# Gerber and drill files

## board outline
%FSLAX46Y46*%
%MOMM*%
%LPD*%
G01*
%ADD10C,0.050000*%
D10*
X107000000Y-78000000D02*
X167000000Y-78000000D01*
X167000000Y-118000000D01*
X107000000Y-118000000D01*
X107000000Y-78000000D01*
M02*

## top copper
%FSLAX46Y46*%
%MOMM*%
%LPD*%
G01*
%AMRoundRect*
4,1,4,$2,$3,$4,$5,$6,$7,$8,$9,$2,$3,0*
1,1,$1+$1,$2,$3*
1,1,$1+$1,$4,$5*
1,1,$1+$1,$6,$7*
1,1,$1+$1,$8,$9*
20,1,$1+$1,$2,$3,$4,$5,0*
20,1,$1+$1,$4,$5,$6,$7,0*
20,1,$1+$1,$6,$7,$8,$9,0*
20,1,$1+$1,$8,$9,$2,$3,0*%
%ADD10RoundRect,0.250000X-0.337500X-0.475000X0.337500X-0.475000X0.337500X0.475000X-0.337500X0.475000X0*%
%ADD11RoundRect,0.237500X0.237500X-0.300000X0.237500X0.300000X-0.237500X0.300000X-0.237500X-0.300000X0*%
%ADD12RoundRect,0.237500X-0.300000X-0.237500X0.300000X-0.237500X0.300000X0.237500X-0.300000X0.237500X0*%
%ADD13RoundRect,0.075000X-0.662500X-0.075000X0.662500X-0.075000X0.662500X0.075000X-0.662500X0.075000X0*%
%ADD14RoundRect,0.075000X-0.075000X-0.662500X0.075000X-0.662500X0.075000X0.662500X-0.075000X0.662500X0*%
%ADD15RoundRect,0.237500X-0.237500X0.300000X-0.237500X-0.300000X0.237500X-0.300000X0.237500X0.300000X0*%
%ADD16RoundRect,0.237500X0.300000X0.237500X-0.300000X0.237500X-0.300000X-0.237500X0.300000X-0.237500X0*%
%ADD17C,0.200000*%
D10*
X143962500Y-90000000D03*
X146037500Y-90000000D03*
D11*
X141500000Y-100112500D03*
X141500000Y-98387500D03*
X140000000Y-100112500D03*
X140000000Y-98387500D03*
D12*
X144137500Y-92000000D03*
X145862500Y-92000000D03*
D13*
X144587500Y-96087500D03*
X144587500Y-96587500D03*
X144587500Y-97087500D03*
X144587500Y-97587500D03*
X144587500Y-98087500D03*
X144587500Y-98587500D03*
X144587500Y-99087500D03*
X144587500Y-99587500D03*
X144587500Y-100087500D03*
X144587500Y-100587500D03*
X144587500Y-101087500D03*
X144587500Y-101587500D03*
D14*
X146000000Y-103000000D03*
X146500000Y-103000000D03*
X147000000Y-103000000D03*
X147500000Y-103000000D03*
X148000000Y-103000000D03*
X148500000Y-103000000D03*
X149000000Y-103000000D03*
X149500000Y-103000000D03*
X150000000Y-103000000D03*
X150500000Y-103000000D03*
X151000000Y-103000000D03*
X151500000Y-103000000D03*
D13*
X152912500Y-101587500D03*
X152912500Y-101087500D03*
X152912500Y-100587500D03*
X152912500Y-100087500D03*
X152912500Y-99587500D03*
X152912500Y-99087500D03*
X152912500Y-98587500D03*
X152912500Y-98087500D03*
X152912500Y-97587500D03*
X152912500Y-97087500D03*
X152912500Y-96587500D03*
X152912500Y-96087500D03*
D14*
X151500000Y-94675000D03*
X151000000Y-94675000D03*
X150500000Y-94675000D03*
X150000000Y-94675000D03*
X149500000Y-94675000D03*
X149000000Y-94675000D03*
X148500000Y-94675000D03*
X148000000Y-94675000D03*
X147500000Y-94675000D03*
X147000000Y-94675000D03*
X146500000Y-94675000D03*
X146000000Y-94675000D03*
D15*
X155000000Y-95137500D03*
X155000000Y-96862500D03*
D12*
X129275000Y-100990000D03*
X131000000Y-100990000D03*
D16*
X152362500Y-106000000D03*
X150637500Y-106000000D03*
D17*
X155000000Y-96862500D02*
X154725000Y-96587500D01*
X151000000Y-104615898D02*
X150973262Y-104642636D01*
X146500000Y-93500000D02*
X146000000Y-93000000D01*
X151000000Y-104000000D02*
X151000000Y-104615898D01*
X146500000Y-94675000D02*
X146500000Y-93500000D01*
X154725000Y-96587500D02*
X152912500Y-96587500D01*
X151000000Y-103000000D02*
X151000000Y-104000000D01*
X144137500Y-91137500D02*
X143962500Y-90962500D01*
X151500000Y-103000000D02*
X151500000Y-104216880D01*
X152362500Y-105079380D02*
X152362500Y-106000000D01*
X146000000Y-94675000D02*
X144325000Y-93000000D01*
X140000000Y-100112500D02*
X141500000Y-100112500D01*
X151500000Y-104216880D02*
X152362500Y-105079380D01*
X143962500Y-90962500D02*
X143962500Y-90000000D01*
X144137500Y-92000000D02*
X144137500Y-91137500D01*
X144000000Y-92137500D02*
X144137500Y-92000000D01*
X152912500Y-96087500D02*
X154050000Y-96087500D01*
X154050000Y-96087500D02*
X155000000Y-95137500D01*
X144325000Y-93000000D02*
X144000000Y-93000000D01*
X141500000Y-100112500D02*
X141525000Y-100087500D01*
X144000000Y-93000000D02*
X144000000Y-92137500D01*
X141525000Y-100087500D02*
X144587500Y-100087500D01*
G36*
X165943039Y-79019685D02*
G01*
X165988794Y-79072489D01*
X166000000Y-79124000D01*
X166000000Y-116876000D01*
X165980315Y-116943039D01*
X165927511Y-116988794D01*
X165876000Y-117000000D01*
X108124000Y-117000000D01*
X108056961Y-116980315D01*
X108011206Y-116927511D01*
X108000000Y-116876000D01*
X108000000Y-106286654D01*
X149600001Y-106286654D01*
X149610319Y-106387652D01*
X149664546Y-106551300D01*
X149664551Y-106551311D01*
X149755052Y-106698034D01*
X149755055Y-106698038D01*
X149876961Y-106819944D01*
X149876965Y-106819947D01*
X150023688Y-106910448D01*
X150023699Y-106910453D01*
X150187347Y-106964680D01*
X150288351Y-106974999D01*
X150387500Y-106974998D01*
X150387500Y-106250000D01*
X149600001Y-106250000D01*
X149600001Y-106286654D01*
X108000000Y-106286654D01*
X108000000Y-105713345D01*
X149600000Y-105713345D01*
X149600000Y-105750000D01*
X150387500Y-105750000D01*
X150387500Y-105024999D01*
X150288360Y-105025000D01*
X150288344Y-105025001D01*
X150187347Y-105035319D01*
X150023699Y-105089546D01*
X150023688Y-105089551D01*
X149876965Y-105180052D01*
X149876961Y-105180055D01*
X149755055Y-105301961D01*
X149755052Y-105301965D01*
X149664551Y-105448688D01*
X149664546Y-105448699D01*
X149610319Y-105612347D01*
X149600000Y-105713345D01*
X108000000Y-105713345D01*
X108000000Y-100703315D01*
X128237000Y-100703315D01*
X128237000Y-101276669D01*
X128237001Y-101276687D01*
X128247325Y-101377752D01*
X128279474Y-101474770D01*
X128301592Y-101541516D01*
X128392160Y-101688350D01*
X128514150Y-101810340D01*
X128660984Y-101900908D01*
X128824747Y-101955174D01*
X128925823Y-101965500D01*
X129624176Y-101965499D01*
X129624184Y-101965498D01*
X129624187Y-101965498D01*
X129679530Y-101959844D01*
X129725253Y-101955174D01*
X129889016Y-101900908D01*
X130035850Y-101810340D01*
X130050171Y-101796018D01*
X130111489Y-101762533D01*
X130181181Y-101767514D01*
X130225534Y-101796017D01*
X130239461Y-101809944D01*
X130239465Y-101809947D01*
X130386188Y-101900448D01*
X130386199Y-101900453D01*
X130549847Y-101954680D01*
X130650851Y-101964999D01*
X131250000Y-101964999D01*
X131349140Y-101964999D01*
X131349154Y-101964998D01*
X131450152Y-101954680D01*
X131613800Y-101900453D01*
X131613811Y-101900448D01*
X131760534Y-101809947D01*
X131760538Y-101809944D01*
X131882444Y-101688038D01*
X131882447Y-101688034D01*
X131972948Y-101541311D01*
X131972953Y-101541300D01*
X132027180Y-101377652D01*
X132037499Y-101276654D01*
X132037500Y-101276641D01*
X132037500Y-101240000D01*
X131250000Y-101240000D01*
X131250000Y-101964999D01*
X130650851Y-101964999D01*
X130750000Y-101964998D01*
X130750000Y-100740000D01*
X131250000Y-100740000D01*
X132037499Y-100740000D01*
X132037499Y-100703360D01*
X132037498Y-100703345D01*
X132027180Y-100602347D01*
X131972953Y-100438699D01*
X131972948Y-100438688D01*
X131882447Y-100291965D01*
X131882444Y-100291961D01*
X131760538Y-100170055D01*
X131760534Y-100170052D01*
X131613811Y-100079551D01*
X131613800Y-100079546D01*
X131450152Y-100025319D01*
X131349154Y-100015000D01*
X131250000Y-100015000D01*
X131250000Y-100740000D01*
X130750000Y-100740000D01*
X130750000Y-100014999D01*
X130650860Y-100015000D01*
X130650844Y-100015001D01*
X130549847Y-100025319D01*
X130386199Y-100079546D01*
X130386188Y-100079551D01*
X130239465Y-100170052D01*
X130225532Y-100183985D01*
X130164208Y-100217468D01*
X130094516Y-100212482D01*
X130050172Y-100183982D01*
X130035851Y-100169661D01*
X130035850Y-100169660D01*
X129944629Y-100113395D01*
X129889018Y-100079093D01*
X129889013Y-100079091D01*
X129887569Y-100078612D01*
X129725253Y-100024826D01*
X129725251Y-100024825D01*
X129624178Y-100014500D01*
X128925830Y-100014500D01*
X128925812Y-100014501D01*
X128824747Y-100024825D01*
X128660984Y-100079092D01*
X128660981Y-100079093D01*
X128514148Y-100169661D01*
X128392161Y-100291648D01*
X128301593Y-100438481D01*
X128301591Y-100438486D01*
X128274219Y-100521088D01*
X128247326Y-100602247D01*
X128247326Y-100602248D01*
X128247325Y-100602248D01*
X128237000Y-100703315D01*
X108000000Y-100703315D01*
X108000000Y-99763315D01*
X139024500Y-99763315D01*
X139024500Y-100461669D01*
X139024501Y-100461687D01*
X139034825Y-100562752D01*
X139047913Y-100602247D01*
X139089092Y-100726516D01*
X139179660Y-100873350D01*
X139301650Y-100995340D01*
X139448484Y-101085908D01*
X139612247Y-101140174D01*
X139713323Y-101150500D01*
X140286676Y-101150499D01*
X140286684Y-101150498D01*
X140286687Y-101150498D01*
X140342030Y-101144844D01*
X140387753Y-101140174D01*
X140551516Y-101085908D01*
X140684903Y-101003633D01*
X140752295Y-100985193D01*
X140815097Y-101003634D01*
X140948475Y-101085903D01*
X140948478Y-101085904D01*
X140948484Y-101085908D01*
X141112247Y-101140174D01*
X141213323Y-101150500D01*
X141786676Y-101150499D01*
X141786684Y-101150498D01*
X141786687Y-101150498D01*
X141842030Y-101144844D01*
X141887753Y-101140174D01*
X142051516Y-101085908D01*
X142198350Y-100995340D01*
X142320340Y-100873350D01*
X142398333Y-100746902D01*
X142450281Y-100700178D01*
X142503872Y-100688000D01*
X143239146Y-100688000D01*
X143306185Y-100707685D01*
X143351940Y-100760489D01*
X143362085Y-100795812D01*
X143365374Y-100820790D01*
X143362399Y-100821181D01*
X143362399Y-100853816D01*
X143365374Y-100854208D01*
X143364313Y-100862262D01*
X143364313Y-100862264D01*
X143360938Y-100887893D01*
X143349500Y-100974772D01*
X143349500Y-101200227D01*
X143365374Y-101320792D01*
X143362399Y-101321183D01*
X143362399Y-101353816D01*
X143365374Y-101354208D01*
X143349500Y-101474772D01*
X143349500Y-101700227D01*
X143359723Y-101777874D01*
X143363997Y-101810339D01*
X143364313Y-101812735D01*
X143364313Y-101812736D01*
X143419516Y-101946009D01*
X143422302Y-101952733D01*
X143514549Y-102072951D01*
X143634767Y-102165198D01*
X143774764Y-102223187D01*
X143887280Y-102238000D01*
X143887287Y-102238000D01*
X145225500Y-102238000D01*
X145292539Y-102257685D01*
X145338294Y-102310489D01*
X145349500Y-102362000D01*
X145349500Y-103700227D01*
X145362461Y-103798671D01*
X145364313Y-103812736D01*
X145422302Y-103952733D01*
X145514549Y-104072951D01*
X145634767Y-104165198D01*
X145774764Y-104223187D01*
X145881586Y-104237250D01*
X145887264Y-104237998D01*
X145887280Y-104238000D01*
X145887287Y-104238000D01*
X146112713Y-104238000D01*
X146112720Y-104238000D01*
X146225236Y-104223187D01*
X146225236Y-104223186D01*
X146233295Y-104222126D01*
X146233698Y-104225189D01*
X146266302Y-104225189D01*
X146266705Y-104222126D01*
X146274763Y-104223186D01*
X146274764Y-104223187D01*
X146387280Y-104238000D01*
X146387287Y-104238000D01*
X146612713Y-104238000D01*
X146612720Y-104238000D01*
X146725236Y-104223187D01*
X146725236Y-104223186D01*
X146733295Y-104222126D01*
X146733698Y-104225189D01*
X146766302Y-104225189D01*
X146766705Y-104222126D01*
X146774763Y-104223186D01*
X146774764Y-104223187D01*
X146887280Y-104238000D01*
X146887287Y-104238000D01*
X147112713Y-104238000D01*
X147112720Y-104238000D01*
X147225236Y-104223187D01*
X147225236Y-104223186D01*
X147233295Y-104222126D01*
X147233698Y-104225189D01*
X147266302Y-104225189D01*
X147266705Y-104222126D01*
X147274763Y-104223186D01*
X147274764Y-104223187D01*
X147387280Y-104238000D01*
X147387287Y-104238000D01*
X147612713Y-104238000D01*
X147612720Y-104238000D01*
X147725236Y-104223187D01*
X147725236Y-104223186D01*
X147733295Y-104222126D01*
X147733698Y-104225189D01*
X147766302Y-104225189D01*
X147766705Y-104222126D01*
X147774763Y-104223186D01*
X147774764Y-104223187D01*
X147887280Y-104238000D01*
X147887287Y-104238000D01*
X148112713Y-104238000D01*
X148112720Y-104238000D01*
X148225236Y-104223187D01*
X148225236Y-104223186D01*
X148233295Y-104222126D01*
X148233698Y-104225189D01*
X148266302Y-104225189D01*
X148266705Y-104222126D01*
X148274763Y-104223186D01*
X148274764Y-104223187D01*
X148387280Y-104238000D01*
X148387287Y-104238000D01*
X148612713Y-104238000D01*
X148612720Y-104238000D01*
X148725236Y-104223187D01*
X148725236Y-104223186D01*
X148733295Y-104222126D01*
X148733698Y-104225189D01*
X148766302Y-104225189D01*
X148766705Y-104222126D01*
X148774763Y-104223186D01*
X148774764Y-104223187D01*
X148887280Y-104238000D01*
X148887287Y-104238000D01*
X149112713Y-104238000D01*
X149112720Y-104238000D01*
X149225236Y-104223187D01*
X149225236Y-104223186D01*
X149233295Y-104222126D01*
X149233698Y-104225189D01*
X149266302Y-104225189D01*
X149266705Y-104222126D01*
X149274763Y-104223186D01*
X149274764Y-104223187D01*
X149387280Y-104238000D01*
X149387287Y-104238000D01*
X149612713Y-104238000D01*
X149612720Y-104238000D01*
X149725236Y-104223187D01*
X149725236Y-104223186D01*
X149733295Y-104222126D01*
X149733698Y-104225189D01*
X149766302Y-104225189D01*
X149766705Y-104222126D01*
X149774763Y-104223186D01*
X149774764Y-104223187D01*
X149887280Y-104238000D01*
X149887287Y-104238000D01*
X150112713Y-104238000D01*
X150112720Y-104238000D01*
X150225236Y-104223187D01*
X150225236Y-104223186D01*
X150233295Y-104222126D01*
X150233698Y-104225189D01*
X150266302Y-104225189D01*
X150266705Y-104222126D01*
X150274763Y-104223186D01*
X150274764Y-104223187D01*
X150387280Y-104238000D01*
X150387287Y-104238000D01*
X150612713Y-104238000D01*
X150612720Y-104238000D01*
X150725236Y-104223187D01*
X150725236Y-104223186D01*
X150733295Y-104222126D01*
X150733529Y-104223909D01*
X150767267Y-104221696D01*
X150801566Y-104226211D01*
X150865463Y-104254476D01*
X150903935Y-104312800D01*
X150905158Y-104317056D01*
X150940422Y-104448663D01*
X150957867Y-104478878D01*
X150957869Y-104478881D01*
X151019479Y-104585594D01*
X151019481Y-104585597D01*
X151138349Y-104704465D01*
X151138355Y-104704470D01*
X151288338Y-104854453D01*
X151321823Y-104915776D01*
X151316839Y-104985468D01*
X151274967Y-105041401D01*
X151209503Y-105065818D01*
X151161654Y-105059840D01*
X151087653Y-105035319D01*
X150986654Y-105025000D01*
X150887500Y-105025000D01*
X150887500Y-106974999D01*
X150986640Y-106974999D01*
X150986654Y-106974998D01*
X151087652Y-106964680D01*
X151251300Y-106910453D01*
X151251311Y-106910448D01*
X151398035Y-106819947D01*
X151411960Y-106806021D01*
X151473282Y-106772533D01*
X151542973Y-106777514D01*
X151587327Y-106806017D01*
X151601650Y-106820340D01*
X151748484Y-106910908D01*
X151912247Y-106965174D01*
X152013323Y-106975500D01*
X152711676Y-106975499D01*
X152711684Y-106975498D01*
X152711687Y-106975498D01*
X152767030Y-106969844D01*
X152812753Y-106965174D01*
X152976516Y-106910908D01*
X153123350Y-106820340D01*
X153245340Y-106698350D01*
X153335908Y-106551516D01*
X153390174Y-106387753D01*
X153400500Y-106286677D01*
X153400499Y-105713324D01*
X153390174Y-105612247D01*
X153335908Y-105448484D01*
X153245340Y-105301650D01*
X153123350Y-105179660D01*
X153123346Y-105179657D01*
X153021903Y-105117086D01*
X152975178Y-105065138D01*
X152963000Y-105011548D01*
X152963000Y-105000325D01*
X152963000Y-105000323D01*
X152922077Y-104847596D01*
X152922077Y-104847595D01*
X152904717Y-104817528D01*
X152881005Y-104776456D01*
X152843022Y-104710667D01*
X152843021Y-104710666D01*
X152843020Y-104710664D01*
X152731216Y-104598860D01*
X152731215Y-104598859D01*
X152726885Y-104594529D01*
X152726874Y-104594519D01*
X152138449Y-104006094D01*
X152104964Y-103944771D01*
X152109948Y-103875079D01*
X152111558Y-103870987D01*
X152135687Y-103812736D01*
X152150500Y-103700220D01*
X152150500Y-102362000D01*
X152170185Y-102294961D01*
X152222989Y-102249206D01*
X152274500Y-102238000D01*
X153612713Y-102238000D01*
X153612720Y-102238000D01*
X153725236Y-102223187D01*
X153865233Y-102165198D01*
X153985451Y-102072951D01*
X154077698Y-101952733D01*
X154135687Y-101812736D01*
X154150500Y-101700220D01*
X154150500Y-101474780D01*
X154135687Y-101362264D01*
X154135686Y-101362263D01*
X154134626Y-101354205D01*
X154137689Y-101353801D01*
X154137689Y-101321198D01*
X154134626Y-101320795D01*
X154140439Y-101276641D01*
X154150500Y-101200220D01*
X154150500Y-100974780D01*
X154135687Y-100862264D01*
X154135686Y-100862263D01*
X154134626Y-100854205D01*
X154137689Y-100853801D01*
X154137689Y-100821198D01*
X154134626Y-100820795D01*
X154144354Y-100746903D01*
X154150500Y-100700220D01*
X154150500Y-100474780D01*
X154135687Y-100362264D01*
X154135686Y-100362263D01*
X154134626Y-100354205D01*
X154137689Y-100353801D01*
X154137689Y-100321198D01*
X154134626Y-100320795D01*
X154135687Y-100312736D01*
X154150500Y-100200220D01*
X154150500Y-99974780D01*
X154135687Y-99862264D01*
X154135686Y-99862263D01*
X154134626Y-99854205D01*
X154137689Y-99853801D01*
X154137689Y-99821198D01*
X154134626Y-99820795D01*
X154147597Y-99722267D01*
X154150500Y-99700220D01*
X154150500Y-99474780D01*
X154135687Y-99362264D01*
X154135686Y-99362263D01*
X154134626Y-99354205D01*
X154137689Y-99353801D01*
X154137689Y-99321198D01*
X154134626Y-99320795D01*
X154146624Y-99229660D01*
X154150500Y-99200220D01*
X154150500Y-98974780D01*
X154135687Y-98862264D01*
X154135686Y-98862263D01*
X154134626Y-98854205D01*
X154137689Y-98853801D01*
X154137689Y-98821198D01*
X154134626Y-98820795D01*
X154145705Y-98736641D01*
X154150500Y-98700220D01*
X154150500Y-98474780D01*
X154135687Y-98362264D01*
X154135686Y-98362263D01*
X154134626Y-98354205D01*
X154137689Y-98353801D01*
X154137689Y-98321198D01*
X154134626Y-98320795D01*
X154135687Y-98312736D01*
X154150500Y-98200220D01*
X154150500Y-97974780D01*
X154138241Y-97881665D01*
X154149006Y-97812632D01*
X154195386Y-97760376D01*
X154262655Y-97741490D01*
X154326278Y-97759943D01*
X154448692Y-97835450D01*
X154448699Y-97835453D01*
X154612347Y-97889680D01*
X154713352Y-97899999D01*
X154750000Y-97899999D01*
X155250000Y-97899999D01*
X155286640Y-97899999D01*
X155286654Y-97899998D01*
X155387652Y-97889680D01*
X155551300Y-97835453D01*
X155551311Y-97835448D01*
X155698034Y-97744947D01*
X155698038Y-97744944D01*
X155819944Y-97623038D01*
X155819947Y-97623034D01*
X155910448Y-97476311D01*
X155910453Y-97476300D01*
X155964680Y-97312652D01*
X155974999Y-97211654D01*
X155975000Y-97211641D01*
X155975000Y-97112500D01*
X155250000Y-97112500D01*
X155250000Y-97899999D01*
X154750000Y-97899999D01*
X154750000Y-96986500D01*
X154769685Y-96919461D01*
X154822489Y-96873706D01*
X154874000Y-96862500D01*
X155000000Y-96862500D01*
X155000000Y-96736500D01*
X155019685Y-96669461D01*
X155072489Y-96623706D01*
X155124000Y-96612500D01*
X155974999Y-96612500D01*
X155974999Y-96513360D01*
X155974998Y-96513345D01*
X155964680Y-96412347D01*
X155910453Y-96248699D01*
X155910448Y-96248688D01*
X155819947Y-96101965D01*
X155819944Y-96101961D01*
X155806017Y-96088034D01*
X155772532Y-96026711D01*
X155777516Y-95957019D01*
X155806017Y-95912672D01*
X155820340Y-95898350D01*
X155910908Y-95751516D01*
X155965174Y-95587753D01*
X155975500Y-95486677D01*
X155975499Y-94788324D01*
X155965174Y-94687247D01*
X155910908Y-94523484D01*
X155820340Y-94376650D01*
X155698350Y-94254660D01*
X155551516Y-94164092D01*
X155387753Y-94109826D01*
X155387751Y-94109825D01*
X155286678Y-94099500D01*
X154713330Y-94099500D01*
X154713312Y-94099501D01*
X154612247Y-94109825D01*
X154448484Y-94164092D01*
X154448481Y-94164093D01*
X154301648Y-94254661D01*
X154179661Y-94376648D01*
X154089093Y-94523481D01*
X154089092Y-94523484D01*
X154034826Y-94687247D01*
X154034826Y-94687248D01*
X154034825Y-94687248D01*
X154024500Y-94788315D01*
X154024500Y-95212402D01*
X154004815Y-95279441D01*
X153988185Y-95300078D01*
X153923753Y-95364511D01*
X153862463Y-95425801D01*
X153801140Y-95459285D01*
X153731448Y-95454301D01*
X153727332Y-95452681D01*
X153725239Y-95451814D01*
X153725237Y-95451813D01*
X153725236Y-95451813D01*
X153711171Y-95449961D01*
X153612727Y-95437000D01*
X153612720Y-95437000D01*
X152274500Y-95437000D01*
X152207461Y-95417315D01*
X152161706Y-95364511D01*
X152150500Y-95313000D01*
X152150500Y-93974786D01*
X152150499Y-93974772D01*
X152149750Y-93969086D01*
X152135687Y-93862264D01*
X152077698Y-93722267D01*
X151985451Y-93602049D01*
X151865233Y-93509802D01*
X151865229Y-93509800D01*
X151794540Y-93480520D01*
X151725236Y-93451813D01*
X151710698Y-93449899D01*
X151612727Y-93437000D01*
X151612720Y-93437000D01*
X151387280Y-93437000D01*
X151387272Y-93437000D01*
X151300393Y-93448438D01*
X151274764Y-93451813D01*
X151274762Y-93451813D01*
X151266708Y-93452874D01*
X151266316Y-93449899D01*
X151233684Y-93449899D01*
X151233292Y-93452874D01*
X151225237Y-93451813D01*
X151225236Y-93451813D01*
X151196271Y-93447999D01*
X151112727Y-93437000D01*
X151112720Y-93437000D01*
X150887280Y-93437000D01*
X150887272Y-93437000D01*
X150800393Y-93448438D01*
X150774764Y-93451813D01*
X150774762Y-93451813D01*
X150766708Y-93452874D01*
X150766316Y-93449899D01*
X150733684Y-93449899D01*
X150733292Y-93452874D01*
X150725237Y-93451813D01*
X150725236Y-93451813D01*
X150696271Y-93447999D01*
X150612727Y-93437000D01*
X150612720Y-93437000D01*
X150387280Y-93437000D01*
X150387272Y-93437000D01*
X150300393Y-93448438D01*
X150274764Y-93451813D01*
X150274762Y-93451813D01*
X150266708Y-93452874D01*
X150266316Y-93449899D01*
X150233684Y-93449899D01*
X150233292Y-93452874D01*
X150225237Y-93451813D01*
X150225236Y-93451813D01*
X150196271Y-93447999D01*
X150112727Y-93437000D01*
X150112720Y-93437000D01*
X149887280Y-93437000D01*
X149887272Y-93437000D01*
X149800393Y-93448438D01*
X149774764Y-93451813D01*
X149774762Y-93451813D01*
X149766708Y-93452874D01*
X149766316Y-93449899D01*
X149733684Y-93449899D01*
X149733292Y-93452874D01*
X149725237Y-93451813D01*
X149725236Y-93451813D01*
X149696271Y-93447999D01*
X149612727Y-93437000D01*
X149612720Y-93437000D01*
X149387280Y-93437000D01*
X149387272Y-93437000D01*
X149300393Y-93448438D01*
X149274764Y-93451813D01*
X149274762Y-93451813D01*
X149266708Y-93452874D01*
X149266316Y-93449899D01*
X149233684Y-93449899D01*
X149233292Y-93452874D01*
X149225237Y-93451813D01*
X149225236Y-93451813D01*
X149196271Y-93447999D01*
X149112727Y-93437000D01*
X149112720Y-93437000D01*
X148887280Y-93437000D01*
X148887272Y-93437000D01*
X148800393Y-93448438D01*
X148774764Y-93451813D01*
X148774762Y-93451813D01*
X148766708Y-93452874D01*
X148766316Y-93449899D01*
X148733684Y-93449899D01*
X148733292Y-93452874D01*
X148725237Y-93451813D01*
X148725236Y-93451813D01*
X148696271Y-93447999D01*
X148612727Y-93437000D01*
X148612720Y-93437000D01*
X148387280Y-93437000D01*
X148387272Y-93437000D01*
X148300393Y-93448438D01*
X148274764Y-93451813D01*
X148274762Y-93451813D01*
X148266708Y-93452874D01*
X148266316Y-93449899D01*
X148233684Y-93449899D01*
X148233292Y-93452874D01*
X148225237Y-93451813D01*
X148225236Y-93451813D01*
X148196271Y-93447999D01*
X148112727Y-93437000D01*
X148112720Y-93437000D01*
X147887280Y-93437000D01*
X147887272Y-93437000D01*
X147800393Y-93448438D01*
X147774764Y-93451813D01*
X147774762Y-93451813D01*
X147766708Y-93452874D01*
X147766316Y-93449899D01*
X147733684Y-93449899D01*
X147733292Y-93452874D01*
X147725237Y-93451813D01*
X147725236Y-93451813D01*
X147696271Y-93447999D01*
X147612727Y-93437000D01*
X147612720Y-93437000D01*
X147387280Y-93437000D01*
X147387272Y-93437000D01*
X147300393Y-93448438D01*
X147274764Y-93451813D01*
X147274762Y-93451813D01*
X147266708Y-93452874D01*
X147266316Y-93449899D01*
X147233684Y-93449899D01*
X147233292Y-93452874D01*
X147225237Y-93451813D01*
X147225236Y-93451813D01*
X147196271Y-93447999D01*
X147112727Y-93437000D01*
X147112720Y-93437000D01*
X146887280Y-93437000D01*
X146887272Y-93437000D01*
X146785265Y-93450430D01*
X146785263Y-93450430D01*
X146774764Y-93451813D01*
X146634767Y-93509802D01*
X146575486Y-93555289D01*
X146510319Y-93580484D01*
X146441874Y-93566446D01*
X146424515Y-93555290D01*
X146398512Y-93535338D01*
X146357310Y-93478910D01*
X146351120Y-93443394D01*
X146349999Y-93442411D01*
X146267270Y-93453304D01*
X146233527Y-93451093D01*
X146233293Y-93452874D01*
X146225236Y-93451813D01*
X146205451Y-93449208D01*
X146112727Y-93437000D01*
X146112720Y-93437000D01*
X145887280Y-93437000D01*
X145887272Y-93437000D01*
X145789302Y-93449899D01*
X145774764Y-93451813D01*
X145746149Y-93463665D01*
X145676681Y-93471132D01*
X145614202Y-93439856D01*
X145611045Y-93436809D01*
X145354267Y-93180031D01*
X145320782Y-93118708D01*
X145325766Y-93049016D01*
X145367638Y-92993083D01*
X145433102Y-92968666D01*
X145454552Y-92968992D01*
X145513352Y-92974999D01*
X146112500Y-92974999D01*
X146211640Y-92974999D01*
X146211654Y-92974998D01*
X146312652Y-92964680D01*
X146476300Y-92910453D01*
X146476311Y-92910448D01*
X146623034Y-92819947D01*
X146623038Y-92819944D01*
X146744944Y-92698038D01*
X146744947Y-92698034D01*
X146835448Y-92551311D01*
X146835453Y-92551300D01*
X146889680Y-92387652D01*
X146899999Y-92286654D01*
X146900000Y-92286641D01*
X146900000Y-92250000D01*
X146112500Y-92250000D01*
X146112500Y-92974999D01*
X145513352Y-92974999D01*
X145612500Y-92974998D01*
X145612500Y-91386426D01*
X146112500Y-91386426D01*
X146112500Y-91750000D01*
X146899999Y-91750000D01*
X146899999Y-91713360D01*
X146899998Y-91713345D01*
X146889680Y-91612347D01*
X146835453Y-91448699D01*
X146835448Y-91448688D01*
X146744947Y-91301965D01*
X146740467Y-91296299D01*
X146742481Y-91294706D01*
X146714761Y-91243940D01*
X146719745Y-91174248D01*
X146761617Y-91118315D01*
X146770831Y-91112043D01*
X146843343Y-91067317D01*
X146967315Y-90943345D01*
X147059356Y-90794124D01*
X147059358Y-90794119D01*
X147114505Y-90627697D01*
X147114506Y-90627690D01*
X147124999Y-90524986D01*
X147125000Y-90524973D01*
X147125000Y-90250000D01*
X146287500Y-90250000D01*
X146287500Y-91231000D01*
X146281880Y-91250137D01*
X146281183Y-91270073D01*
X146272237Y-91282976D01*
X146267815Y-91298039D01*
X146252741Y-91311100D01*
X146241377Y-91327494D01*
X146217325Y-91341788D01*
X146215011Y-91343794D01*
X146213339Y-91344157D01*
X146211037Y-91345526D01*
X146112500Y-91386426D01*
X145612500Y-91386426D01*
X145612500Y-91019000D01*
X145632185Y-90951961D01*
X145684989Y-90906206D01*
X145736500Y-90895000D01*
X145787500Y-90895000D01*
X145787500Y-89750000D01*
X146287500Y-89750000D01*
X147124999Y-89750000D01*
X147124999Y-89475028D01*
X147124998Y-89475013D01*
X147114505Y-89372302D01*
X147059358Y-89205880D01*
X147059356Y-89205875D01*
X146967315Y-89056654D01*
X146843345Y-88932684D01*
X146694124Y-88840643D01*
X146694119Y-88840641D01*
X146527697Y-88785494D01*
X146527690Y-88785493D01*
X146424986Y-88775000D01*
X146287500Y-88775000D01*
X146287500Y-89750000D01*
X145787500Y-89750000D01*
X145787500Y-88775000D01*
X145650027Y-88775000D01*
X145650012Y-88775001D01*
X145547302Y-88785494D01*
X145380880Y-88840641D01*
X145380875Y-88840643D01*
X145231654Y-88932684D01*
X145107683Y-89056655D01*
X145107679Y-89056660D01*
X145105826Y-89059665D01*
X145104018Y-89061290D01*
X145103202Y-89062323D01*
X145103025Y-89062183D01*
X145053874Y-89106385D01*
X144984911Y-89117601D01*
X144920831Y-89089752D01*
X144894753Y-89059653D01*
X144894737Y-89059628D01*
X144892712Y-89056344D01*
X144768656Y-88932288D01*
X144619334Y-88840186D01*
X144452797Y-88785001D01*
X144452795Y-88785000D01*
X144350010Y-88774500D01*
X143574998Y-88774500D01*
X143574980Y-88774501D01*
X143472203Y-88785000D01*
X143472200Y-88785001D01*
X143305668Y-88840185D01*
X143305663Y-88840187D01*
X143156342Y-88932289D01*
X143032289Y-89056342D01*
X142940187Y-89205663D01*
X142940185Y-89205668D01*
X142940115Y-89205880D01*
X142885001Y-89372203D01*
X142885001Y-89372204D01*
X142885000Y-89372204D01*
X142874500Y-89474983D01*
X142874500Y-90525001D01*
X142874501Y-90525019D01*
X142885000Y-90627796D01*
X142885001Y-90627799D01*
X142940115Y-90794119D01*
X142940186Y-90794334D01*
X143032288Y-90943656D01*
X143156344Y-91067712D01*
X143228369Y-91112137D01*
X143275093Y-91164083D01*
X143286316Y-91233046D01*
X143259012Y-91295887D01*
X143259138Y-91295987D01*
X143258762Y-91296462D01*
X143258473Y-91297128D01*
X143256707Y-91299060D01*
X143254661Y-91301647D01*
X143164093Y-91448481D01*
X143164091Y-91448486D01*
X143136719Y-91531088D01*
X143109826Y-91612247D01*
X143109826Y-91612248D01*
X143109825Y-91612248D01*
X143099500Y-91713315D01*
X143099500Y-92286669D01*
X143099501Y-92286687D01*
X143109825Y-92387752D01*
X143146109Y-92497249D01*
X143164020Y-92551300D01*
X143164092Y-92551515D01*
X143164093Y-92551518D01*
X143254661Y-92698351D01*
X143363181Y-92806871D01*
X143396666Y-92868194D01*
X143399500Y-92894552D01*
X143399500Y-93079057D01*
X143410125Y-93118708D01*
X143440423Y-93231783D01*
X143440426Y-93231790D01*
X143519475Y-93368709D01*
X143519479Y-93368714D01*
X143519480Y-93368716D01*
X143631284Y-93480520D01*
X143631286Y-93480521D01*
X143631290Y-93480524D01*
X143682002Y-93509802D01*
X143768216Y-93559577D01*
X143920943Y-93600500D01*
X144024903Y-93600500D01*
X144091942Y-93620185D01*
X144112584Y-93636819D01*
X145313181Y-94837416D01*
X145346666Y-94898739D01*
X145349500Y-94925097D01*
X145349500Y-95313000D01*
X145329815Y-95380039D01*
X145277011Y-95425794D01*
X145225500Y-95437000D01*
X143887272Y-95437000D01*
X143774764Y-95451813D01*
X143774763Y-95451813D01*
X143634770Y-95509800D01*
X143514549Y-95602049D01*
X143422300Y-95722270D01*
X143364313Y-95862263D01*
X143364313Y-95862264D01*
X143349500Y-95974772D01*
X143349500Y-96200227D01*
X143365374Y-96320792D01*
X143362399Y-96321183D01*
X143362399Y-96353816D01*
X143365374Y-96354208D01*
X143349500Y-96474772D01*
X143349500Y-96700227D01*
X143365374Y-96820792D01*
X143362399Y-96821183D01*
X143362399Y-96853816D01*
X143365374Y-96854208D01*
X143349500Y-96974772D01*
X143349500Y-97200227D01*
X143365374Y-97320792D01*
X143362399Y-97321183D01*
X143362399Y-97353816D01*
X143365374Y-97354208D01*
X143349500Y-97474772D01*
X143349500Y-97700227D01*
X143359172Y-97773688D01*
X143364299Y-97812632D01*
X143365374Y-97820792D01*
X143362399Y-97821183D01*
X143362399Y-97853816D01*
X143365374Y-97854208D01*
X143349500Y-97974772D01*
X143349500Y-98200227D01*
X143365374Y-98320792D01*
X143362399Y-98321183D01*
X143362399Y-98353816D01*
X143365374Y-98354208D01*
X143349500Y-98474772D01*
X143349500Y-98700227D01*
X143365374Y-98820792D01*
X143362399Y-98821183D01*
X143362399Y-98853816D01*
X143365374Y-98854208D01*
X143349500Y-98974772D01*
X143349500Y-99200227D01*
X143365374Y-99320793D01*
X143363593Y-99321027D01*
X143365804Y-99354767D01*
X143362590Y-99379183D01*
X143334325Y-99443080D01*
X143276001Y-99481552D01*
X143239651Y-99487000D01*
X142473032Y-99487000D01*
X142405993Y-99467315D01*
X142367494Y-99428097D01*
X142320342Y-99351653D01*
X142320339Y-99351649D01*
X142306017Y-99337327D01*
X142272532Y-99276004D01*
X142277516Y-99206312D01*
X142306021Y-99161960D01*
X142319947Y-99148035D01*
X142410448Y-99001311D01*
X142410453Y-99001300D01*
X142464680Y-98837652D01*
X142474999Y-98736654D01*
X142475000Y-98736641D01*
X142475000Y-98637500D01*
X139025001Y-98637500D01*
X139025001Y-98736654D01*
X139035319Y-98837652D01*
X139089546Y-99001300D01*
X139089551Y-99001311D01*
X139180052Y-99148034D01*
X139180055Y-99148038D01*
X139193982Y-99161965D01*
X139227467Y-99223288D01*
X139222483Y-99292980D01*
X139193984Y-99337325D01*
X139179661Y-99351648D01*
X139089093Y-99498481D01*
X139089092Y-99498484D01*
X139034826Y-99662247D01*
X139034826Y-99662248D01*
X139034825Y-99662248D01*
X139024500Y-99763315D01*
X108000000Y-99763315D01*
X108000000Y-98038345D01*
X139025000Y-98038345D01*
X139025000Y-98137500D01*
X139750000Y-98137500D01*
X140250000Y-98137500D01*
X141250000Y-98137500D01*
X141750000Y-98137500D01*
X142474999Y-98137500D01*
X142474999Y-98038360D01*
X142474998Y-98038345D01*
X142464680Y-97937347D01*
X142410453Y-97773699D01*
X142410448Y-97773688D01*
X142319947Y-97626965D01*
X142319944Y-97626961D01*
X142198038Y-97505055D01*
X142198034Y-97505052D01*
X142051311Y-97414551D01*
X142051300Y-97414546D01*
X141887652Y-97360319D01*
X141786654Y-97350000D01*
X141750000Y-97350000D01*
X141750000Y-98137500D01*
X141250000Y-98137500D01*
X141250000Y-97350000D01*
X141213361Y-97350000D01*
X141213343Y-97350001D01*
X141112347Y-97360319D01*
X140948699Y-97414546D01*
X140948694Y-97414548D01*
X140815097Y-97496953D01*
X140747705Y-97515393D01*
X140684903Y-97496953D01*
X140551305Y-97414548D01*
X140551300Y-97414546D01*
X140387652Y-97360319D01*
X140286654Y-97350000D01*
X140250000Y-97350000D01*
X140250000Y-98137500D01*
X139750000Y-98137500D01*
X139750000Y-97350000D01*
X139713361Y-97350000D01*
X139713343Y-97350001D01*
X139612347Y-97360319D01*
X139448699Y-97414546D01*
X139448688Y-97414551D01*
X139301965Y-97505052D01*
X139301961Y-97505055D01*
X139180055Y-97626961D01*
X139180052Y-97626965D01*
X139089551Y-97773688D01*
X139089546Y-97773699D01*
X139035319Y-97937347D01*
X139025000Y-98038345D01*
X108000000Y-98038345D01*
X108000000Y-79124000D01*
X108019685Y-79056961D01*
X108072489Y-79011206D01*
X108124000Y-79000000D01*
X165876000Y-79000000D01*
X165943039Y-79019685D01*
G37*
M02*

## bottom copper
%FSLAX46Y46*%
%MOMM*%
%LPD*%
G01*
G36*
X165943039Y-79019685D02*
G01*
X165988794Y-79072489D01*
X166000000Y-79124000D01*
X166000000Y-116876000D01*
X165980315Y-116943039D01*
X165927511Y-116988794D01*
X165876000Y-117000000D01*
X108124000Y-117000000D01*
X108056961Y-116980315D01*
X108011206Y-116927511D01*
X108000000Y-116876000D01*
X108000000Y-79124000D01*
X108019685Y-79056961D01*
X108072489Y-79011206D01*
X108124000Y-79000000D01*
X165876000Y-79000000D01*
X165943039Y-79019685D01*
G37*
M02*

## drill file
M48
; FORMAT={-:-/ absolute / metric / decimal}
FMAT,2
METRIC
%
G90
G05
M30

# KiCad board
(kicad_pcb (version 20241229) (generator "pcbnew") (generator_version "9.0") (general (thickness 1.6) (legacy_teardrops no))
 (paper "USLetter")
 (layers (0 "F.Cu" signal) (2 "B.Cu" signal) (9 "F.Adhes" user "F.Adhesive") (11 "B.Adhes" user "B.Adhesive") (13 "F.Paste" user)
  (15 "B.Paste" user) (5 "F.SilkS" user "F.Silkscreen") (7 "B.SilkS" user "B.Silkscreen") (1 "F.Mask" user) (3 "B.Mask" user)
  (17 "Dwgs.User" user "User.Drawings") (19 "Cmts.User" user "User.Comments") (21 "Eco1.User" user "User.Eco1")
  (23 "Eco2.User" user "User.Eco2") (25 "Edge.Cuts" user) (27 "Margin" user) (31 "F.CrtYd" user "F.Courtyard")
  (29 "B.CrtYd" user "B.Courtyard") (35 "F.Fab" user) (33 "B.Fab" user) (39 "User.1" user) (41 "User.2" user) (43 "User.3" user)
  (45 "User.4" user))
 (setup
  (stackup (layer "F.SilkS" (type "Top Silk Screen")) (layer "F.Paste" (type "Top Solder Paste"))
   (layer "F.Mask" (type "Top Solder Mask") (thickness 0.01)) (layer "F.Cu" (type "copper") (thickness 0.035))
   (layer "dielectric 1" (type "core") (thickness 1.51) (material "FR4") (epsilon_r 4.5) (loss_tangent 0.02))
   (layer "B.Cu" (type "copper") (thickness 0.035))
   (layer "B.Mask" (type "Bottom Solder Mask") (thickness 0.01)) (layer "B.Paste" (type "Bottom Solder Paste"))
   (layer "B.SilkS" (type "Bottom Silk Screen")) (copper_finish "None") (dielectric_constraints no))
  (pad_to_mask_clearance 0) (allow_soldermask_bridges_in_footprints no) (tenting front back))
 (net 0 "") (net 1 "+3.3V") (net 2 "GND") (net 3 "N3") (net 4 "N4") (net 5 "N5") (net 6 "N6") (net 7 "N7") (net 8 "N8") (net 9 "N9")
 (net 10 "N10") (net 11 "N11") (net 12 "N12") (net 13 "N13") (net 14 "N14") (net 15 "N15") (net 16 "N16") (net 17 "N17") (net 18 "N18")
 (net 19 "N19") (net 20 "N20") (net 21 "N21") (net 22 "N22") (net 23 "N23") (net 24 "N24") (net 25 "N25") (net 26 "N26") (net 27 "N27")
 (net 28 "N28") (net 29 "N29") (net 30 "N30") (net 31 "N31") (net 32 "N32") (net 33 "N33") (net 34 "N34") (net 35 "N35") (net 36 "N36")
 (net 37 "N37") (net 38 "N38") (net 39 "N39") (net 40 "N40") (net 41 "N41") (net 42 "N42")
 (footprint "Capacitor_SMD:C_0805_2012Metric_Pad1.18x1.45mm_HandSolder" (layer "F.Cu") (at 145 90)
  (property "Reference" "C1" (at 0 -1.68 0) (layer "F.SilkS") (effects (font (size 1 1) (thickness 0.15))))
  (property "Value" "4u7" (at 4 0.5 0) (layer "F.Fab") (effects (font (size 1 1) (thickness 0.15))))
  (pad "1" smd roundrect (at -1.0375 0) (size 1.175 1.45) (layers "F.Cu" "F.Mask" "F.Paste") (roundrect_rratio 0.212766) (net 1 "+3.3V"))
  (pad "2" smd roundrect (at 1.0375 0) (size 1.175 1.45) (layers "F.Cu" "F.Mask" "F.Paste") (roundrect_rratio 0.212766) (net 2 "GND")))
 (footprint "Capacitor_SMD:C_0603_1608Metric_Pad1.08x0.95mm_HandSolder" (layer "F.Cu") (at 141.5 99.25 90)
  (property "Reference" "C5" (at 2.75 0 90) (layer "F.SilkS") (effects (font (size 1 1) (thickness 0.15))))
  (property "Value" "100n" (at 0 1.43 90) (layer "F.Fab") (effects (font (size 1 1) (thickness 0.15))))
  (pad "1" smd roundrect (at -0.8625 0 90) (size 1.075 0.95) (layers "F.Cu" "F.Mask" "F.Paste") (roundrect_rratio 0.25) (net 1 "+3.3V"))
  (pad "2" smd roundrect (at 0.8625 0 90) (size 1.075 0.95) (layers "F.Cu" "F.Mask" "F.Paste") (roundrect_rratio 0.25) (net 2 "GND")))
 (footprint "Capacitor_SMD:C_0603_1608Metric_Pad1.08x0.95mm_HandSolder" (layer "F.Cu") (at 140 99.25 90)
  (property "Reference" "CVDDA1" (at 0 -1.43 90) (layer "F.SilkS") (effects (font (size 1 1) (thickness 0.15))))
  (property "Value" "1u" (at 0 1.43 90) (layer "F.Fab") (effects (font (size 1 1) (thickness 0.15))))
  (pad "1" smd roundrect (at -0.8625 0 90) (size 1.075 0.95) (layers "F.Cu" "F.Mask" "F.Paste") (roundrect_rratio 0.25) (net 1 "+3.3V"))
  (pad "2" smd roundrect (at 0.8625 0 90) (size 1.075 0.95) (layers "F.Cu" "F.Mask" "F.Paste") (roundrect_rratio 0.25) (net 2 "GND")))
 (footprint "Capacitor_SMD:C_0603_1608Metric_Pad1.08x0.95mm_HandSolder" (layer "F.Cu") (at 145 92)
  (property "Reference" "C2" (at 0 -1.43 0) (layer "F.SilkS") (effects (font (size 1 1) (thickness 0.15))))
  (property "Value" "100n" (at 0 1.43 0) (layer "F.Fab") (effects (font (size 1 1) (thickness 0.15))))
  (pad "1" smd roundrect (at -0.8625 0) (size 1.075 0.95) (layers "F.Cu" "F.Mask" "F.Paste") (roundrect_rratio 0.25) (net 1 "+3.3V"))
  (pad "2" smd roundrect (at 0.8625 0) (size 1.075 0.95) (layers "F.Cu" "F.Mask" "F.Paste") (roundrect_rratio 0.25) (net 2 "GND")))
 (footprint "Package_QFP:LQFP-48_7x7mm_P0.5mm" (layer "F.Cu") (at 148.75 98.8375)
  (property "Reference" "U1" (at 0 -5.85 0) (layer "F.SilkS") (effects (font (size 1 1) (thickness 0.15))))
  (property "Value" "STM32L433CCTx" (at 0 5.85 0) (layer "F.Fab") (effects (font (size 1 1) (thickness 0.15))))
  (pad "1" smd roundrect (at -4.1625 -2.75) (size 1.475 0.3) (layers "F.Cu" "F.Mask" "F.Paste") (roundrect_rratio 0.25) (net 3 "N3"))
  (pad "2" smd roundrect (at -4.1625 -2.25) (size 1.475 0.3) (layers "F.Cu" "F.Mask" "F.Paste") (roundrect_rratio 0.25) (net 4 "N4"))
  (pad "3" smd roundrect (at -4.1625 -1.75) (size 1.475 0.3) (layers "F.Cu" "F.Mask" "F.Paste") (roundrect_rratio 0.25) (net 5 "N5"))
  (pad "4" smd roundrect (at -4.1625 -1.25) (size 1.475 0.3) (layers "F.Cu" "F.Mask" "F.Paste") (roundrect_rratio 0.25) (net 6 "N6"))
  (pad "5" smd roundrect (at -4.1625 -0.75) (size 1.475 0.3) (layers "F.Cu" "F.Mask" "F.Paste") (roundrect_rratio 0.25) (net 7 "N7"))
  (pad "6" smd roundrect (at -4.1625 -0.25) (size 1.475 0.3) (layers "F.Cu" "F.Mask" "F.Paste") (roundrect_rratio 0.25) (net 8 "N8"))
  (pad "7" smd roundrect (at -4.1625 0.25) (size 1.475 0.3) (layers "F.Cu" "F.Mask" "F.Paste") (roundrect_rratio 0.25) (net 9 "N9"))
  (pad "8" smd roundrect (at -4.1625 0.75) (size 1.475 0.3) (layers "F.Cu" "F.Mask" "F.Paste") (roundrect_rratio 0.25) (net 2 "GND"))
  (pad "9" smd roundrect (at -4.1625 1.25) (size 1.475 0.3) (layers "F.Cu" "F.Mask" "F.Paste") (roundrect_rratio 0.25) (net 1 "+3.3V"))
  (pad "10" smd roundrect (at -4.1625 1.75) (size 1.475 0.3) (layers "F.Cu" "F.Mask" "F.Paste") (roundrect_rratio 0.25) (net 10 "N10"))
  (pad "11" smd roundrect (at -4.1625 2.25) (size 1.475 0.3) (layers "F.Cu" "F.Mask" "F.Paste") (roundrect_rratio 0.25) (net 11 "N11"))
  (pad "12" smd roundrect (at -4.1625 2.75) (size 1.475 0.3) (layers "F.Cu" "F.Mask" "F.Paste") (roundrect_rratio 0.25) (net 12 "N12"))
  (pad "13" smd roundrect (at -2.75 4.1625) (size 0.3 1.475) (layers "F.Cu" "F.Mask" "F.Paste") (roundrect_rratio 0.25) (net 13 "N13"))
  (pad "14" smd roundrect (at -2.25 4.1625) (size 0.3 1.475) (layers "F.Cu" "F.Mask" "F.Paste") (roundrect_rratio 0.25) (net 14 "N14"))
  (pad "15" smd roundrect (at -1.75 4.1625) (size 0.3 1.475) (layers "F.Cu" "F.Mask" "F.Paste") (roundrect_rratio 0.25) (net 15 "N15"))
  (pad "16" smd roundrect (at -1.25 4.1625) (size 0.3 1.475) (layers "F.Cu" "F.Mask" "F.Paste") (roundrect_rratio 0.25) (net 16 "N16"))
  (pad "17" smd roundrect (at -0.75 4.1625) (size 0.3 1.475) (layers "F.Cu" "F.Mask" "F.Paste") (roundrect_rratio 0.25) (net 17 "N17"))
  (pad "18" smd roundrect (at -0.25 4.1625) (size 0.3 1.475) (layers "F.Cu" "F.Mask" "F.Paste") (roundrect_rratio 0.25) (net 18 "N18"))
  (pad "19" smd roundrect (at 0.25 4.1625) (size 0.3 1.475) (layers "F.Cu" "F.Mask" "F.Paste") (roundrect_rratio 0.25) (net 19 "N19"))
  (pad "20" smd roundrect (at 0.75 4.1625) (size 0.3 1.475) (layers "F.Cu" "F.Mask" "F.Paste") (roundrect_rratio 0.25) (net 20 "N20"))
  (pad "21" smd roundrect (at 1.25 4.1625) (size 0.3 1.475) (layers "F.Cu" "F.Mask" "F.Paste") (roundrect_rratio 0.25) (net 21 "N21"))
  (pad "22" smd roundrect (at 1.75 4.1625) (size 0.3 1.475) (layers "F.Cu" "F.Mask" "F.Paste") (roundrect_rratio 0.25) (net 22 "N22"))
  (pad "23" smd roundrect (at 2.25 4.1625) (size 0.3 1.475) (layers "F.Cu" "F.Mask" "F.Paste") (roundrect_rratio 0.25) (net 2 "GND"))
  (pad "24" smd roundrect (at 2.75 4.1625) (size 0.3 1.475) (layers "F.Cu" "F.Mask" "F.Paste") (roundrect_rratio 0.25) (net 1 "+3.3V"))
  (pad "25" smd roundrect (at 4.1625 2.75) (size 1.475 0.3) (layers "F.Cu" "F.Mask" "F.Paste") (roundrect_rratio 0.25) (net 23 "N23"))
  (pad "26" smd roundrect (at 4.1625 2.25) (size 1.475 0.3) (layers "F.Cu" "F.Mask" "F.Paste") (roundrect_rratio 0.25) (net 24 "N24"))
  (pad "27" smd roundrect (at 4.1625 1.75) (size 1.475 0.3) (layers "F.Cu" "F.Mask" "F.Paste") (roundrect_rratio 0.25) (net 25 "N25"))
  (pad "28" smd roundrect (at 4.1625 1.25) (size 1.475 0.3) (layers "F.Cu" "F.Mask" "F.Paste") (roundrect_rratio 0.25) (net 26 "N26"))
  (pad "29" smd roundrect (at 4.1625 0.75) (size 1.475 0.3) (layers "F.Cu" "F.Mask" "F.Paste") (roundrect_rratio 0.25) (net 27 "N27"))
  (pad "30" smd roundrect (at 4.1625 0.25) (size 1.475 0.3) (layers "F.Cu" "F.Mask" "F.Paste") (roundrect_rratio 0.25) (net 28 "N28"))
  (pad "31" smd roundrect (at 4.1625 -0.25) (size 1.475 0.3) (layers "F.Cu" "F.Mask" "F.Paste") (roundrect_rratio 0.25) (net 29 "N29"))
  (pad "32" smd roundrect (at 4.1625 -0.75) (size 1.475 0.3) (layers "F.Cu" "F.Mask" "F.Paste") (roundrect_rratio 0.25) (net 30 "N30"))
  (pad "33" smd roundrect (at 4.1625 -1.25) (size 1.475 0.3) (layers "F.Cu" "F.Mask" "F.Paste") (roundrect_rratio 0.25) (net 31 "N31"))
  (pad "34" smd roundrect (at 4.1625 -1.75) (size 1.475 0.3) (layers "F.Cu" "F.Mask" "F.Paste") (roundrect_rratio 0.25) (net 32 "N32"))
  (pad "35" smd roundrect (at 4.1625 -2.25) (size 1.475 0.3) (layers "F.Cu" "F.Mask" "F.Paste") (roundrect_rratio 0.25) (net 2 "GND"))
  (pad "36" smd roundrect (at 4.1625 -2.75) (size 1.475 0.3) (layers "F.Cu" "F.Mask" "F.Paste") (roundrect_rratio 0.25) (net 1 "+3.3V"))
  (pad "37" smd roundrect (at 2.75 -4.1625) (size 0.3 1.475) (layers "F.Cu" "F.Mask" "F.Paste") (roundrect_rratio 0.25) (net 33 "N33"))
  (pad "38" smd roundrect (at 2.25 -4.1625) (size 0.3 1.475) (layers "F.Cu" "F.Mask" "F.Paste") (roundrect_rratio 0.25) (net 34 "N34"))
  (pad "39" smd roundrect (at 1.75 -4.1625) (size 0.3 1.475) (layers "F.Cu" "F.Mask" "F.Paste") (roundrect_rratio 0.25) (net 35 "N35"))
  (pad "40" smd roundrect (at 1.25 -4.1625) (size 0.3 1.475) (layers "F.Cu" "F.Mask" "F.Paste") (roundrect_rratio 0.25) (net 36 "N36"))
  (pad "41" smd roundrect (at 0.75 -4.1625) (size 0.3 1.475) (layers "F.Cu" "F.Mask" "F.Paste") (roundrect_rratio 0.25) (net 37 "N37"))
  (pad "42" smd roundrect (at 0.25 -4.1625) (size 0.3 1.475) (layers "F.Cu" "F.Mask" "F.Paste") (roundrect_rratio 0.25) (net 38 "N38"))
  (pad "43" smd roundrect (at -0.25 -4.1625) (size 0.3 1.475) (layers "F.Cu" "F.Mask" "F.Paste") (roundrect_rratio 0.25) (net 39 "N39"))
  (pad "44" smd roundrect (at -0.75 -4.1625) (size 0.3 1.475) (layers "F.Cu" "F.Mask" "F.Paste") (roundrect_rratio 0.25) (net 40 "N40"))
  (pad "45" smd roundrect (at -1.25 -4.1625) (size 0.3 1.475) (layers "F.Cu" "F.Mask" "F.Paste") (roundrect_rratio 0.25) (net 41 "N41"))
  (pad "46" smd roundrect (at -1.75 -4.1625) (size 0.3 1.475) (layers "F.Cu" "F.Mask" "F.Paste") (roundrect_rratio 0.25) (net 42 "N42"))
  (pad "47" smd roundrect (at -2.25 -4.1625) (size 0.3 1.475) (layers "F.Cu" "F.Mask" "F.Paste") (roundrect_rratio 0.25) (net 2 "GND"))
  (pad "48" smd roundrect (at -2.75 -4.1625) (size 0.3 1.475) (layers "F.Cu" "F.Mask" "F.Paste") (roundrect_rratio 0.25) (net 1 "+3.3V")))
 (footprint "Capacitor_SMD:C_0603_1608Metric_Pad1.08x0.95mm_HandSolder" (layer "F.Cu") (at 155 96 -90)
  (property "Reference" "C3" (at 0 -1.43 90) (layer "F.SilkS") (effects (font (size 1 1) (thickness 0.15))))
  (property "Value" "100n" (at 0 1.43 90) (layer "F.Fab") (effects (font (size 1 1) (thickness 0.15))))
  (pad "1" smd roundrect (at -0.8625 0 270) (size 1.075 0.95) (layers "F.Cu" "F.Mask" "F.Paste") (roundrect_rratio 0.25) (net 1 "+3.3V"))
  (pad "2" smd roundrect (at 0.8625 0 270) (size 1.075 0.95) (layers "F.Cu" "F.Mask" "F.Paste") (roundrect_rratio 0.25) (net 2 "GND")))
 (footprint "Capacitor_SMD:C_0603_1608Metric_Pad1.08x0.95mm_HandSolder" (layer "F.Cu") (at 130.1375 100.99)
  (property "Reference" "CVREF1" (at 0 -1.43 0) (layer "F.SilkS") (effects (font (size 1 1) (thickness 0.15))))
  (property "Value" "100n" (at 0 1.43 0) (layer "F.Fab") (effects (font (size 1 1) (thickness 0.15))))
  (pad "1" smd roundrect (at -0.8625 0) (size 1.075 0.95) (layers "F.Cu" "F.Mask" "F.Paste") (roundrect_rratio 0.25) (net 1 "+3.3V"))
  (pad "2" smd roundrect (at 0.8625 0) (size 1.075 0.95) (layers "F.Cu" "F.Mask" "F.Paste") (roundrect_rratio 0.25) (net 2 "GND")))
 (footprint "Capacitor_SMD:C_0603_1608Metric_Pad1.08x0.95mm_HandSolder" (layer "F.Cu") (at 151.5 106 180)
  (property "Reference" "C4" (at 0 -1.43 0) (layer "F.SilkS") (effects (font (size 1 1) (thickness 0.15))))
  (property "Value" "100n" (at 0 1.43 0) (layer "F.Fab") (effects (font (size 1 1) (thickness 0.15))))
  (pad "1" smd roundrect (at -0.8625 0 180) (size 1.075 0.95) (layers "F.Cu" "F.Mask" "F.Paste") (roundrect_rratio 0.25) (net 1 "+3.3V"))
  (pad "2" smd roundrect (at 0.8625 0 180) (size 1.075 0.95) (layers "F.Cu" "F.Mask" "F.Paste") (roundrect_rratio 0.25) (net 2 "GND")))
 (gr_rect (start 107 78) (end 167 118) (stroke (width 0.05) (type default)) (fill no) (layer "Edge.Cuts"))
 (segment (start 155 96.8625) (end 154.725 96.5875) (width 0.2) (layer "F.Cu") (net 2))
 (segment (start 151 104.615898) (end 150.973262 104.642636) (width 0.2) (layer "F.Cu") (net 2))
 (segment (start 146.5 93.5) (end 146 93) (width 0.2) (layer "F.Cu") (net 2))
 (segment (start 151 104) (end 151 104.615898) (width 0.2) (layer "F.Cu") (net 2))
 (segment (start 146.5 94.675) (end 146.5 93.5) (width 0.2) (layer "F.Cu") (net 2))
 (segment (start 154.725 96.5875) (end 152.9125 96.5875) (width 0.2) (layer "F.Cu") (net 2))
 (segment (start 151 103) (end 151 104) (width 0.2) (layer "F.Cu") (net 2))
 (segment (start 144.1375 91.1375) (end 143.9625 90.9625) (width 0.2) (layer "F.Cu") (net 1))
 (segment (start 151.5 103) (end 151.5 104.21688) (width 0.2) (layer "F.Cu") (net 1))
 (segment (start 152.3625 105.07938) (end 152.3625 106) (width 0.2) (layer "F.Cu") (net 1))
 (segment (start 146 94.675) (end 144.325 93) (width 0.2) (layer "F.Cu") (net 1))
 (segment (start 140 100.1125) (end 141.5 100.1125) (width 0.2) (layer "F.Cu") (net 1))
 (segment (start 151.5 104.21688) (end 152.3625 105.07938) (width 0.2) (layer "F.Cu") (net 1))
 (segment (start 143.9625 90.9625) (end 143.9625 90) (width 0.2) (layer "F.Cu") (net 1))
 (segment (start 144.1375 92) (end 144.1375 91.1375) (width 0.2) (layer "F.Cu") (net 1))
 (segment (start 144 92.1375) (end 144.1375 92) (width 0.2) (layer "F.Cu") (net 1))
 (segment (start 152.9125 96.0875) (end 154.05 96.0875) (width 0.2) (layer "F.Cu") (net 1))
 (segment (start 154.05 96.0875) (end 155 95.1375) (width 0.2) (layer "F.Cu") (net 1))
 (segment (start 144.325 93) (end 144 93) (width 0.2) (layer "F.Cu") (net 1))
 (segment (start 141.5 100.1125) (end 141.525 100.0875) (width 0.2) (layer "F.Cu") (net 1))
 (segment (start 144 93) (end 144 92.1375) (width 0.2) (layer "F.Cu") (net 1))
 (segment (start 141.525 100.0875) (end 144.5875 100.0875) (width 0.2) (layer "F.Cu") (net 1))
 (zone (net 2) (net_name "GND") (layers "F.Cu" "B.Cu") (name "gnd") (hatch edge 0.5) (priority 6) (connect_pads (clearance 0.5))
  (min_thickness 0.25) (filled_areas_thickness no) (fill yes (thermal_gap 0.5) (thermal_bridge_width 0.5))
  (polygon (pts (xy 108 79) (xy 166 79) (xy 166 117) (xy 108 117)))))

